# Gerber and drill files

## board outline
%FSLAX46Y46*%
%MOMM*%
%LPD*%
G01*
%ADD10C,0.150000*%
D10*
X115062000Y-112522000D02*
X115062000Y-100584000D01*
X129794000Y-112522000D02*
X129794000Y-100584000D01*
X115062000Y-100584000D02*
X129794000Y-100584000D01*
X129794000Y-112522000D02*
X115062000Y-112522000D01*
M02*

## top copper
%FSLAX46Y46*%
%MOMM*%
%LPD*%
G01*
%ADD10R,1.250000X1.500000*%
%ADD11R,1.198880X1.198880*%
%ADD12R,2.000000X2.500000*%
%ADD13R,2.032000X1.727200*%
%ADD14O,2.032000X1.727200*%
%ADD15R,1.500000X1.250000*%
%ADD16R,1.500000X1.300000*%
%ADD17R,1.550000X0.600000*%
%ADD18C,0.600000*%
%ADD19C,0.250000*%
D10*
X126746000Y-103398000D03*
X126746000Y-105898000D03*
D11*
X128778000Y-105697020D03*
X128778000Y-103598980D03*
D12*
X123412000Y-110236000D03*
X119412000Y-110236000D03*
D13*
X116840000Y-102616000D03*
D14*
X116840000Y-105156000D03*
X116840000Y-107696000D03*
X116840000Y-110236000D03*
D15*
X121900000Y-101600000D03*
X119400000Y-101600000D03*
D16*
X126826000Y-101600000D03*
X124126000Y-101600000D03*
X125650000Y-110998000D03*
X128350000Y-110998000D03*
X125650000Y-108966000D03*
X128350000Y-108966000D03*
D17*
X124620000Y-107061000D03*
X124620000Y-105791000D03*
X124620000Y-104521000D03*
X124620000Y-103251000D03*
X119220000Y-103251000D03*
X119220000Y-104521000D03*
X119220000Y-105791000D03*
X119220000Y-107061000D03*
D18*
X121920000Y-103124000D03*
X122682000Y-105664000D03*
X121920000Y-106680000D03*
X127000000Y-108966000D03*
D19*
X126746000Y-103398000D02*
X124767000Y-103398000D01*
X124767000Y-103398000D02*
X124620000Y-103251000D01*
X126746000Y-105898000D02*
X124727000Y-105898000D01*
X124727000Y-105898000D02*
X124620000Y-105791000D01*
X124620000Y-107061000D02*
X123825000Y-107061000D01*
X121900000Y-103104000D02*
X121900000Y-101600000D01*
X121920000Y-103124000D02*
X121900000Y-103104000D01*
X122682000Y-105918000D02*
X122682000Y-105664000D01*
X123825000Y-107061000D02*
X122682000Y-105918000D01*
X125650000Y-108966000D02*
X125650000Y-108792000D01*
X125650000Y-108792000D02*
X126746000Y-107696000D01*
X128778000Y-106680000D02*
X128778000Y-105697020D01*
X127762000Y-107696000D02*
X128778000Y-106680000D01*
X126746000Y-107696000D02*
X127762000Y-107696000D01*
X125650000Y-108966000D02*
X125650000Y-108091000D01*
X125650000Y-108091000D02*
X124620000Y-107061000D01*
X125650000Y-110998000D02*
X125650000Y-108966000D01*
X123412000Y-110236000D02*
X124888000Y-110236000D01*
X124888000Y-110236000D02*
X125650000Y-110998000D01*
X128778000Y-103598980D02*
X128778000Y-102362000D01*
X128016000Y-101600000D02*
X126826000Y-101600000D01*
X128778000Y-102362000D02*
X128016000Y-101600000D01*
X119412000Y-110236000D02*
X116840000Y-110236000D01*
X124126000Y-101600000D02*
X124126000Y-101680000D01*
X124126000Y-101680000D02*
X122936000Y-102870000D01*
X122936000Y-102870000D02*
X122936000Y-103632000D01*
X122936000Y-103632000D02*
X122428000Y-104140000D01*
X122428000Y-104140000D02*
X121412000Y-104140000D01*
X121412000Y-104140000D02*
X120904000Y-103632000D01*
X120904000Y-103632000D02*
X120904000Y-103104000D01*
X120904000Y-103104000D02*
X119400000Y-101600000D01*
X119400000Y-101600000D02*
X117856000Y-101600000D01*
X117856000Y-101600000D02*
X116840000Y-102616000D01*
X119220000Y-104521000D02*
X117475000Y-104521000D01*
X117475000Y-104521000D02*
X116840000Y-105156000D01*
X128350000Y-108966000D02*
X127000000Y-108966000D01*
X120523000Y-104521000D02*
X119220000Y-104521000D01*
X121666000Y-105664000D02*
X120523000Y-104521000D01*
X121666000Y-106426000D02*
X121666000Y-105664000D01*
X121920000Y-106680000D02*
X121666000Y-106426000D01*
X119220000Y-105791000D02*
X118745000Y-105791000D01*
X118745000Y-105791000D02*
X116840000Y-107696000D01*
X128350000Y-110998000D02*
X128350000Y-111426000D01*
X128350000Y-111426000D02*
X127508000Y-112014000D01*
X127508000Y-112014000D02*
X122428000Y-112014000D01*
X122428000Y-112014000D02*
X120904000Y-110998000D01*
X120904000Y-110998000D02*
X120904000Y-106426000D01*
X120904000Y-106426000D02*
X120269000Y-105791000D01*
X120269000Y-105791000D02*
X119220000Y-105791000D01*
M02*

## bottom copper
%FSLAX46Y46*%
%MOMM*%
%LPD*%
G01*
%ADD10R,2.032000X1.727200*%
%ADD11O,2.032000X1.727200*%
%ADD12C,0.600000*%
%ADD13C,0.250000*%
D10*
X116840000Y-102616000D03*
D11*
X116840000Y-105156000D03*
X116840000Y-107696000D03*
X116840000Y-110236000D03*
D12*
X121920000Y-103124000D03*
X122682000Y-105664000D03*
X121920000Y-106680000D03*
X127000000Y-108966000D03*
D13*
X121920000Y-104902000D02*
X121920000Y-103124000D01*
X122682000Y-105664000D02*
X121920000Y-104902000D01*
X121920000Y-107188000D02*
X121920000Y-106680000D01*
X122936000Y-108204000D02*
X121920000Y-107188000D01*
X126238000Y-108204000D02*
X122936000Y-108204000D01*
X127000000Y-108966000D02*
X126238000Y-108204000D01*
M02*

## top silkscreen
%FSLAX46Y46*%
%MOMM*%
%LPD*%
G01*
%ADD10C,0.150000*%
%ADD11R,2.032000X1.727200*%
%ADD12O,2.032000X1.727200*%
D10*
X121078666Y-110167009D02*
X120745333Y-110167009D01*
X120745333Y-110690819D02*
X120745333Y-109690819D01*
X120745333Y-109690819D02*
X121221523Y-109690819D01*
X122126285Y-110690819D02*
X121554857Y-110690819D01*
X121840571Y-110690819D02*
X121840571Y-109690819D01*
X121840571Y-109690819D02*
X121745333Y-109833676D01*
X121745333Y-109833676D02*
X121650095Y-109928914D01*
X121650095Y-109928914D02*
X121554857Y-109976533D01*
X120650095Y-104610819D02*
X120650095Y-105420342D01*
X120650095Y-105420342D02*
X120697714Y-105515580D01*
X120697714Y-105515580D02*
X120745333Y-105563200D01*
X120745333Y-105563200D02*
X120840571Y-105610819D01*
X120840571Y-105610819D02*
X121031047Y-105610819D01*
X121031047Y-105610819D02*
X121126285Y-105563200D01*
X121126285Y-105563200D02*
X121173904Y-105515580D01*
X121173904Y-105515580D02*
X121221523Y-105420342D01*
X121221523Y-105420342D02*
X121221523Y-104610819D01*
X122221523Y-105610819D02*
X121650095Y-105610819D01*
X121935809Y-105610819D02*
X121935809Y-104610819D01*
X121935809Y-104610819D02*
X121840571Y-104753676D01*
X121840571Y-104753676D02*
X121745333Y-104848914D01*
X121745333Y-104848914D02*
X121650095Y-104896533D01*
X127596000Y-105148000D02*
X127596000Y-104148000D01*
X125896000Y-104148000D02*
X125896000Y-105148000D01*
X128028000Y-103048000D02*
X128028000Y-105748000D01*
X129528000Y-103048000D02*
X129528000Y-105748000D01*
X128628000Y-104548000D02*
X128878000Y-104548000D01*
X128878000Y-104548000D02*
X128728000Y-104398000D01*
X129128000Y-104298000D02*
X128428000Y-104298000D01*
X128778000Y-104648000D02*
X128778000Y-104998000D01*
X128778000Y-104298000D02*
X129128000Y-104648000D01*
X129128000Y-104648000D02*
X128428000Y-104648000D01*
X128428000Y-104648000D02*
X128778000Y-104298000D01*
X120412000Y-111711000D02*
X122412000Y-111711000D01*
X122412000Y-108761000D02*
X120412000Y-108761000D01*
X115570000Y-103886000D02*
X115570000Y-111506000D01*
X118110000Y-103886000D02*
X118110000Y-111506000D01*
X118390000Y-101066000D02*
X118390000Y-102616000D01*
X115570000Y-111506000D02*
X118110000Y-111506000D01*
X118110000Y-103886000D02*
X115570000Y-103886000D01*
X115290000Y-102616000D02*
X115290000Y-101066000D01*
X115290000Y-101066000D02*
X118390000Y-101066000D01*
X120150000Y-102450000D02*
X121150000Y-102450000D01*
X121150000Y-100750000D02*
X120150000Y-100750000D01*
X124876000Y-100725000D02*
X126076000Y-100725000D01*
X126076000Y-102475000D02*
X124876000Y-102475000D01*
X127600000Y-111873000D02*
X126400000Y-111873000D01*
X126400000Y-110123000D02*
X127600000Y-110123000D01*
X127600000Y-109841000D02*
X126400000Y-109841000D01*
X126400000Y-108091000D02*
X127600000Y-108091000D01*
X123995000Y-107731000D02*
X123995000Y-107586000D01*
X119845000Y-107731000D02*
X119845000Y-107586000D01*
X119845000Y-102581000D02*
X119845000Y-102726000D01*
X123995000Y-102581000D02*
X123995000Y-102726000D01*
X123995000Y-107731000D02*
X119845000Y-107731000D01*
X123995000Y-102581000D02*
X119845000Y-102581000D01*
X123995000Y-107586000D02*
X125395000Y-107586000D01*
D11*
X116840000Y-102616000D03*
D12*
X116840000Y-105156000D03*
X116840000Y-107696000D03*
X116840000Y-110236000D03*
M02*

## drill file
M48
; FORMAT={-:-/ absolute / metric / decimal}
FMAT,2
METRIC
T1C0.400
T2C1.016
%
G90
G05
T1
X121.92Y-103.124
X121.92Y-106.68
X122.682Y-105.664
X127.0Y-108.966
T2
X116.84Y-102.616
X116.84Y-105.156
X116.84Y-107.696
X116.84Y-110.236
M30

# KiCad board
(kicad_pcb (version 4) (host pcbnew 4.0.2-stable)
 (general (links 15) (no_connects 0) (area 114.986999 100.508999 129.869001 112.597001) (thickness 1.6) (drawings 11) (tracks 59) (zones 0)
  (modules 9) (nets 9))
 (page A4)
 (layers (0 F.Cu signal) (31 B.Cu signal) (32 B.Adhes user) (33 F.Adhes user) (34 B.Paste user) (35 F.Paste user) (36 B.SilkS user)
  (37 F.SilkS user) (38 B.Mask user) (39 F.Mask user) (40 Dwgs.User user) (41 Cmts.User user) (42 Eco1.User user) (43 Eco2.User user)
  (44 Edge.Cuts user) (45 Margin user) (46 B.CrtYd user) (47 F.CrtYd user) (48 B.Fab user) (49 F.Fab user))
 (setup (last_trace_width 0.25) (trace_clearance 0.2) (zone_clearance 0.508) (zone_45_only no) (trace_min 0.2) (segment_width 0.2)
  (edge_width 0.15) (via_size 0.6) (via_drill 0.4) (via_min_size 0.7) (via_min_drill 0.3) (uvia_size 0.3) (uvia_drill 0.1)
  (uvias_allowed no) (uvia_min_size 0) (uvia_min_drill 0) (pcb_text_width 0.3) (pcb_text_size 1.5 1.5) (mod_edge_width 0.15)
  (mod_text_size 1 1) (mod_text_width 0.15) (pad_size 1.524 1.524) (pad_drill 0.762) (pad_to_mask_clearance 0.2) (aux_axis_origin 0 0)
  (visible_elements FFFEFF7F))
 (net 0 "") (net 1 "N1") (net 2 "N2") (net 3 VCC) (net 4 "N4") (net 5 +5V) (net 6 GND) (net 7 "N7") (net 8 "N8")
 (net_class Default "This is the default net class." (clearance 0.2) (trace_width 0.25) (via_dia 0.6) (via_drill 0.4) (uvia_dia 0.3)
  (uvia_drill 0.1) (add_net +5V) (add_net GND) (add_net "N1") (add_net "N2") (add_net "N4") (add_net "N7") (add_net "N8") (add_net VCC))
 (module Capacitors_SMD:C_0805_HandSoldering (layer F.Cu) (at 126.746 104.648 270)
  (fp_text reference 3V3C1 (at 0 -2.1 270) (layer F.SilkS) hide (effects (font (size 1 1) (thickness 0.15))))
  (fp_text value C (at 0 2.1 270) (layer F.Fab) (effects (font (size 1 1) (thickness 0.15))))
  (fp_line (start 0.5 -0.85) (end -0.5 -0.85) (layer F.SilkS) (width 0.15))
  (fp_line (start -0.5 0.85) (end 0.5 0.85) (layer F.SilkS) (width 0.15))
  (pad 1 smd rect (at -1.25 0 270) (size 1.5 1.25) (layers F.Cu F.Paste F.Mask) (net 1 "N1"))
  (pad 2 smd rect (at 1.25 0 270) (size 1.5 1.25) (layers F.Cu F.Paste F.Mask) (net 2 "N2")))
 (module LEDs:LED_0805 (layer F.Cu) (at 128.778 104.648 270)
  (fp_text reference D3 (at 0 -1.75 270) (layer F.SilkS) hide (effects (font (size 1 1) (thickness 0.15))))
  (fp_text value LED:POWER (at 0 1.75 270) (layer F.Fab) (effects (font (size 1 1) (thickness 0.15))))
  (fp_line (start -1.6 0.75) (end 1.1 0.75) (layer F.SilkS) (width 0.15))
  (fp_line (start -1.6 -0.75) (end 1.1 -0.75) (layer F.SilkS) (width 0.15))
  (fp_line (start -0.1 0.15) (end -0.1 -0.1) (layer F.SilkS) (width 0.15))
  (fp_line (start -0.1 -0.1) (end -0.25 0.05) (layer F.SilkS) (width 0.15))
  (fp_line (start -0.35 -0.35) (end -0.35 0.35) (layer F.SilkS) (width 0.15))
  (fp_line (start 0 0) (end 0.35 0) (layer F.SilkS) (width 0.15))
  (fp_line (start -0.35 0) (end 0 -0.35) (layer F.SilkS) (width 0.15))
  (fp_line (start 0 -0.35) (end 0 0.35) (layer F.SilkS) (width 0.15))
  (fp_line (start 0 0.35) (end -0.35 0) (layer F.SilkS) (width 0.15))
  (pad 2 smd rect (at 1.04902 0 90) (size 1.19888 1.19888) (layers F.Cu F.Paste F.Mask) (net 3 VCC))
  (pad 1 smd rect (at -1.04902 0 90) (size 1.19888 1.19888) (layers F.Cu F.Paste F.Mask) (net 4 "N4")))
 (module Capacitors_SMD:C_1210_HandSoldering (layer F.Cu) (at 121.412 110.236 180)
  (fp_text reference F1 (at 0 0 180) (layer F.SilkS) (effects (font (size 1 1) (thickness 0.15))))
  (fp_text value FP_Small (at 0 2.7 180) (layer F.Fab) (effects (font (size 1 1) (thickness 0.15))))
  (fp_line (start 1 -1.475) (end -1 -1.475) (layer F.SilkS) (width 0.15))
  (fp_line (start -1 1.475) (end 1 1.475) (layer F.SilkS) (width 0.15))
  (pad 1 smd rect (at -2 0 180) (size 2 2.5) (layers F.Cu F.Paste F.Mask) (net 3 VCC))
  (pad 2 smd rect (at 2 0 180) (size 2 2.5) (layers F.Cu F.Paste F.Mask) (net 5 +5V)))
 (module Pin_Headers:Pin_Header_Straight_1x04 (layer F.Cu) (at 116.84 102.616)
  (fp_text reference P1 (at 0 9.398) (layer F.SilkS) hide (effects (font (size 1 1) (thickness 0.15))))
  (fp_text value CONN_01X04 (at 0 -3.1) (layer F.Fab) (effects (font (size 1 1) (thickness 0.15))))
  (fp_line (start -1.27 1.27) (end -1.27 8.89) (layer F.SilkS) (width 0.15))
  (fp_line (start 1.27 1.27) (end 1.27 8.89) (layer F.SilkS) (width 0.15))
  (fp_line (start 1.55 -1.55) (end 1.55 0) (layer F.SilkS) (width 0.15))
  (fp_line (start -1.27 8.89) (end 1.27 8.89) (layer F.SilkS) (width 0.15))
  (fp_line (start 1.27 1.27) (end -1.27 1.27) (layer F.SilkS) (width 0.15))
  (fp_line (start -1.55 0) (end -1.55 -1.55) (layer F.SilkS) (width 0.15))
  (fp_line (start -1.55 -1.55) (end 1.55 -1.55) (layer F.SilkS) (width 0.15))
  (pad 1 thru_hole rect (at 0 0) (size 2.032 1.7272) (drill 1.016) (layers *.Cu *.Mask F.SilkS) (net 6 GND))
  (pad 2 thru_hole oval (at 0 2.54) (size 2.032 1.7272) (drill 1.016) (layers *.Cu *.Mask F.SilkS) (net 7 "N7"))
  (pad 3 thru_hole oval (at 0 5.08) (size 2.032 1.7272) (drill 1.016) (layers *.Cu *.Mask F.SilkS) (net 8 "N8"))
  (pad 4 thru_hole oval (at 0 7.62) (size 2.032 1.7272) (drill 1.016) (layers *.Cu *.Mask F.SilkS) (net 5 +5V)))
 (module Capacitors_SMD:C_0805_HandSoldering (layer F.Cu) (at 120.65 101.6 180)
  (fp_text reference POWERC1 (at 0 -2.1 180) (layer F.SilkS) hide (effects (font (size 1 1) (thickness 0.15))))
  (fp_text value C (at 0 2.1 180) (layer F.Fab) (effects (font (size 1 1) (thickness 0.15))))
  (fp_line (start 0.5 -0.85) (end -0.5 -0.85) (layer F.SilkS) (width 0.15))
  (fp_line (start -0.5 0.85) (end 0.5 0.85) (layer F.SilkS) (width 0.15))
  (pad 1 smd rect (at -1.25 0 180) (size 1.5 1.25) (layers F.Cu F.Paste F.Mask) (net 3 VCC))
  (pad 2 smd rect (at 1.25 0 180) (size 1.5 1.25) (layers F.Cu F.Paste F.Mask) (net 6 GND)))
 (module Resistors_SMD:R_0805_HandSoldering (layer F.Cu) (at 125.476 101.6 180)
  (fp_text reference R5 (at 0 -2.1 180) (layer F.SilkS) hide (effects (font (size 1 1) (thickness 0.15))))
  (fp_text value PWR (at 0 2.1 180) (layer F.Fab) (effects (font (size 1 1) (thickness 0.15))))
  (fp_line (start 0.6 0.875) (end -0.6 0.875) (layer F.SilkS) (width 0.15))
  (fp_line (start -0.6 -0.875) (end 0.6 -0.875) (layer F.SilkS) (width 0.15))
  (pad 1 smd rect (at -1.35 0 180) (size 1.5 1.3) (layers F.Cu F.Paste F.Mask) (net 4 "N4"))
  (pad 2 smd rect (at 1.35 0 180) (size 1.5 1.3) (layers F.Cu F.Paste F.Mask) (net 6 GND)))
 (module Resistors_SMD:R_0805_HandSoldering (layer F.Cu) (at 127 110.998)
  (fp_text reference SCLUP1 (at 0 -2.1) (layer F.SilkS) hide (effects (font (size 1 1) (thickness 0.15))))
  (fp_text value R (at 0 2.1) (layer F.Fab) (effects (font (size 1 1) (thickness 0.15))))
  (fp_line (start 0.6 0.875) (end -0.6 0.875) (layer F.SilkS) (width 0.15))
  (fp_line (start -0.6 -0.875) (end 0.6 -0.875) (layer F.SilkS) (width 0.15))
  (pad 1 smd rect (at -1.35 0) (size 1.5 1.3) (layers F.Cu F.Paste F.Mask) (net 3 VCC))
  (pad 2 smd rect (at 1.35 0) (size 1.5 1.3) (layers F.Cu F.Paste F.Mask) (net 8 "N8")))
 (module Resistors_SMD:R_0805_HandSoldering (layer F.Cu) (at 127 108.966)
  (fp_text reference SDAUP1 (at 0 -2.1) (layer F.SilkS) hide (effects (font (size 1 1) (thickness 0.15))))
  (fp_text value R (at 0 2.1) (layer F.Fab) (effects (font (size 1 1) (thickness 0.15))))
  (fp_line (start 0.6 0.875) (end -0.6 0.875) (layer F.SilkS) (width 0.15))
  (fp_line (start -0.6 -0.875) (end 0.6 -0.875) (layer F.SilkS) (width 0.15))
  (pad 1 smd rect (at -1.35 0) (size 1.5 1.3) (layers F.Cu F.Paste F.Mask) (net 3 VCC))
  (pad 2 smd rect (at 1.35 0) (size 1.5 1.3) (layers F.Cu F.Paste F.Mask) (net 7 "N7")))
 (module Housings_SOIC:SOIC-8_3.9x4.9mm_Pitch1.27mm (layer F.Cu) (at 121.92 105.156 180)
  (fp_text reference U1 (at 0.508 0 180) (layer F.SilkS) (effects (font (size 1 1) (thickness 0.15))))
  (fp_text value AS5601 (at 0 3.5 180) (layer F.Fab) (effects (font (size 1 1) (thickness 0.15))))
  (fp_line (start -2.075 -2.575) (end -2.075 -2.43) (layer F.SilkS) (width 0.15))
  (fp_line (start 2.075 -2.575) (end 2.075 -2.43) (layer F.SilkS) (width 0.15))
  (fp_line (start 2.075 2.575) (end 2.075 2.43) (layer F.SilkS) (width 0.15))
  (fp_line (start -2.075 2.575) (end -2.075 2.43) (layer F.SilkS) (width 0.15))
  (fp_line (start -2.075 -2.575) (end 2.075 -2.575) (layer F.SilkS) (width 0.15))
  (fp_line (start -2.075 2.575) (end 2.075 2.575) (layer F.SilkS) (width 0.15))
  (fp_line (start -2.075 -2.43) (end -3.475 -2.43) (layer F.SilkS) (width 0.15))
  (pad 1 smd rect (at -2.7 -1.905 180) (size 1.55 0.6) (layers F.Cu F.Paste F.Mask) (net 3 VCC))
  (pad 2 smd rect (at -2.7 -0.635 180) (size 1.55 0.6) (layers F.Cu F.Paste F.Mask) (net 2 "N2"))
  (pad 3 smd rect (at -2.7 0.635 180) (size 1.55 0.6) (layers F.Cu F.Paste F.Mask))
  (pad 4 smd rect (at -2.7 1.905 180) (size 1.55 0.6) (layers F.Cu F.Paste F.Mask) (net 1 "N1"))
  (pad 5 smd rect (at 2.7 1.905 180) (size 1.55 0.6) (layers F.Cu F.Paste F.Mask))
  (pad 6 smd rect (at 2.7 0.635 180) (size 1.55 0.6) (layers F.Cu F.Paste F.Mask) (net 7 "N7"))
  (pad 7 smd rect (at 2.7 -0.635 180) (size 1.55 0.6) (layers F.Cu F.Paste F.Mask) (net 8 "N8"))
  (pad 8 smd rect (at 2.7 -1.905 180) (size 1.55 0.6) (layers F.Cu F.Paste F.Mask)))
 (gr_line (start 115.062 112.522) (end 115.062 100.584) (angle 90) (layer Edge.Cuts) (width 0.15))
 (gr_line (start 129.794 112.522) (end 129.794 100.584) (angle 90) (layer Edge.Cuts) (width 0.15))
 (gr_line (start 115.062 100.584) (end 129.794 100.584) (angle 90) (layer Edge.Cuts) (width 0.15))
 (gr_line (start 129.794 112.522) (end 115.062 112.522) (angle 90) (layer Edge.Cuts) (width 0.15))
 (segment (start 126.746 103.398) (end 124.767 103.398) (width 0.25) (layer F.Cu) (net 1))
 (segment (start 124.767 103.398) (end 124.62 103.251) (width 0.25) (layer F.Cu) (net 1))
 (segment (start 126.746 105.898) (end 124.727 105.898) (width 0.25) (layer F.Cu) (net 2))
 (segment (start 124.727 105.898) (end 124.62 105.791) (width 0.25) (layer F.Cu) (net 2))
 (segment (start 124.62 107.061) (end 123.825 107.061) (width 0.25) (layer F.Cu) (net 3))
 (segment (start 121.9 103.104) (end 121.9 101.6) (width 0.25) (layer F.Cu) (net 3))
 (segment (start 121.92 103.124) (end 121.9 103.104) (width 0.25) (layer F.Cu) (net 3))
 (via (at 121.92 103.124) (size 0.6) (drill 0.4) (layers F.Cu B.Cu) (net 3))
 (segment (start 121.92 104.902) (end 121.92 103.124) (width 0.25) (layer B.Cu) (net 3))
 (segment (start 122.682 105.664) (end 121.92 104.902) (width 0.25) (layer B.Cu) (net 3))
 (via (at 122.682 105.664) (size 0.6) (drill 0.4) (layers F.Cu B.Cu) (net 3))
 (segment (start 122.682 105.918) (end 122.682 105.664) (width 0.25) (layer F.Cu) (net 3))
 (segment (start 123.825 107.061) (end 122.682 105.918) (width 0.25) (layer F.Cu) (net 3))
 (segment (start 125.65 108.966) (end 125.65 108.792) (width 0.25) (layer F.Cu) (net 3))
 (segment (start 125.65 108.792) (end 126.746 107.696) (width 0.25) (layer F.Cu) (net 3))
 (segment (start 128.778 106.68) (end 128.778 105.69702) (width 0.25) (layer F.Cu) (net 3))
 (segment (start 127.762 107.696) (end 128.778 106.68) (width 0.25) (layer F.Cu) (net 3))
 (segment (start 126.746 107.696) (end 127.762 107.696) (width 0.25) (layer F.Cu) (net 3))
 (segment (start 125.65 108.966) (end 125.65 108.091) (width 0.25) (layer F.Cu) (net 3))
 (segment (start 125.65 108.091) (end 124.62 107.061) (width 0.25) (layer F.Cu) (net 3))
 (segment (start 125.65 110.998) (end 125.65 108.966) (width 0.25) (layer F.Cu) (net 3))
 (segment (start 123.412 110.236) (end 124.888 110.236) (width 0.25) (layer F.Cu) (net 3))
 (segment (start 124.888 110.236) (end 125.65 110.998) (width 0.25) (layer F.Cu) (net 3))
 (segment (start 128.778 103.59898) (end 128.778 102.362) (width 0.25) (layer F.Cu) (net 4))
 (segment (start 128.016 101.6) (end 126.826 101.6) (width 0.25) (layer F.Cu) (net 4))
 (segment (start 128.778 102.362) (end 128.016 101.6) (width 0.25) (layer F.Cu) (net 4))
 (segment (start 119.412 110.236) (end 116.84 110.236) (width 0.25) (layer F.Cu) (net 5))
 (segment (start 124.126 101.6) (end 124.126 101.68) (width 0.25) (layer F.Cu) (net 6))
 (segment (start 124.126 101.68) (end 122.936 102.87) (width 0.25) (layer F.Cu) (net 6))
 (segment (start 122.936 102.87) (end 122.936 103.632) (width 0.25) (layer F.Cu) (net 6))
 (segment (start 122.936 103.632) (end 122.428 104.14) (width 0.25) (layer F.Cu) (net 6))
 (segment (start 122.428 104.14) (end 121.412 104.14) (width 0.25) (layer F.Cu) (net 6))
 (segment (start 121.412 104.14) (end 120.904 103.632) (width 0.25) (layer F.Cu) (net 6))
 (segment (start 120.904 103.632) (end 120.904 103.104) (width 0.25) (layer F.Cu) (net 6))
 (segment (start 120.904 103.104) (end 119.4 101.6) (width 0.25) (layer F.Cu) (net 6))
 (segment (start 119.4 101.6) (end 117.856 101.6) (width 0.25) (layer F.Cu) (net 6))
 (segment (start 117.856 101.6) (end 116.84 102.616) (width 0.25) (layer F.Cu) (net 6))
 (segment (start 119.22 104.521) (end 117.475 104.521) (width 0.25) (layer F.Cu) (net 7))
 (segment (start 117.475 104.521) (end 116.84 105.156) (width 0.25) (layer F.Cu) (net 7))
 (segment (start 128.35 108.966) (end 127 108.966) (width 0.25) (layer F.Cu) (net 7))
 (segment (start 120.523 104.521) (end 119.22 104.521) (width 0.25) (layer F.Cu) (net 7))
 (segment (start 121.666 105.664) (end 120.523 104.521) (width 0.25) (layer F.Cu) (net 7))
 (segment (start 121.666 106.426) (end 121.666 105.664) (width 0.25) (layer F.Cu) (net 7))
 (segment (start 121.92 106.68) (end 121.666 106.426) (width 0.25) (layer F.Cu) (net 7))
 (via (at 121.92 106.68) (size 0.6) (drill 0.4) (layers F.Cu B.Cu) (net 7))
 (segment (start 121.92 107.188) (end 121.92 106.68) (width 0.25) (layer B.Cu) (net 7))
 (segment (start 122.936 108.204) (end 121.92 107.188) (width 0.25) (layer B.Cu) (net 7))
 (segment (start 126.238 108.204) (end 122.936 108.204) (width 0.25) (layer B.Cu) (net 7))
 (segment (start 127 108.966) (end 126.238 108.204) (width 0.25) (layer B.Cu) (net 7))
 (via (at 127 108.966) (size 0.6) (drill 0.4) (layers F.Cu B.Cu) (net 7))
 (segment (start 119.22 105.791) (end 118.745 105.791) (width 0.25) (layer F.Cu) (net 8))
 (segment (start 118.745 105.791) (end 116.84 107.696) (width 0.25) (layer F.Cu) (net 8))
 (segment (start 128.35 110.998) (end 128.35 111.426) (width 0.25) (layer F.Cu) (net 8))
 (segment (start 128.35 111.426) (end 127.508 112.014) (width 0.25) (layer F.Cu) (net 8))
 (segment (start 127.508 112.014) (end 122.428 112.014) (width 0.25) (layer F.Cu) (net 8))
 (segment (start 122.428 112.014) (end 120.904 110.998) (width 0.25) (layer F.Cu) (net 8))
 (segment (start 120.904 110.998) (end 120.904 106.426) (width 0.25) (layer F.Cu) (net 8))
 (segment (start 120.904 106.426) (end 120.269 105.791) (width 0.25) (layer F.Cu) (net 8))
 (segment (start 120.269 105.791) (end 119.22 105.791) (width 0.25) (layer F.Cu) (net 8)))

